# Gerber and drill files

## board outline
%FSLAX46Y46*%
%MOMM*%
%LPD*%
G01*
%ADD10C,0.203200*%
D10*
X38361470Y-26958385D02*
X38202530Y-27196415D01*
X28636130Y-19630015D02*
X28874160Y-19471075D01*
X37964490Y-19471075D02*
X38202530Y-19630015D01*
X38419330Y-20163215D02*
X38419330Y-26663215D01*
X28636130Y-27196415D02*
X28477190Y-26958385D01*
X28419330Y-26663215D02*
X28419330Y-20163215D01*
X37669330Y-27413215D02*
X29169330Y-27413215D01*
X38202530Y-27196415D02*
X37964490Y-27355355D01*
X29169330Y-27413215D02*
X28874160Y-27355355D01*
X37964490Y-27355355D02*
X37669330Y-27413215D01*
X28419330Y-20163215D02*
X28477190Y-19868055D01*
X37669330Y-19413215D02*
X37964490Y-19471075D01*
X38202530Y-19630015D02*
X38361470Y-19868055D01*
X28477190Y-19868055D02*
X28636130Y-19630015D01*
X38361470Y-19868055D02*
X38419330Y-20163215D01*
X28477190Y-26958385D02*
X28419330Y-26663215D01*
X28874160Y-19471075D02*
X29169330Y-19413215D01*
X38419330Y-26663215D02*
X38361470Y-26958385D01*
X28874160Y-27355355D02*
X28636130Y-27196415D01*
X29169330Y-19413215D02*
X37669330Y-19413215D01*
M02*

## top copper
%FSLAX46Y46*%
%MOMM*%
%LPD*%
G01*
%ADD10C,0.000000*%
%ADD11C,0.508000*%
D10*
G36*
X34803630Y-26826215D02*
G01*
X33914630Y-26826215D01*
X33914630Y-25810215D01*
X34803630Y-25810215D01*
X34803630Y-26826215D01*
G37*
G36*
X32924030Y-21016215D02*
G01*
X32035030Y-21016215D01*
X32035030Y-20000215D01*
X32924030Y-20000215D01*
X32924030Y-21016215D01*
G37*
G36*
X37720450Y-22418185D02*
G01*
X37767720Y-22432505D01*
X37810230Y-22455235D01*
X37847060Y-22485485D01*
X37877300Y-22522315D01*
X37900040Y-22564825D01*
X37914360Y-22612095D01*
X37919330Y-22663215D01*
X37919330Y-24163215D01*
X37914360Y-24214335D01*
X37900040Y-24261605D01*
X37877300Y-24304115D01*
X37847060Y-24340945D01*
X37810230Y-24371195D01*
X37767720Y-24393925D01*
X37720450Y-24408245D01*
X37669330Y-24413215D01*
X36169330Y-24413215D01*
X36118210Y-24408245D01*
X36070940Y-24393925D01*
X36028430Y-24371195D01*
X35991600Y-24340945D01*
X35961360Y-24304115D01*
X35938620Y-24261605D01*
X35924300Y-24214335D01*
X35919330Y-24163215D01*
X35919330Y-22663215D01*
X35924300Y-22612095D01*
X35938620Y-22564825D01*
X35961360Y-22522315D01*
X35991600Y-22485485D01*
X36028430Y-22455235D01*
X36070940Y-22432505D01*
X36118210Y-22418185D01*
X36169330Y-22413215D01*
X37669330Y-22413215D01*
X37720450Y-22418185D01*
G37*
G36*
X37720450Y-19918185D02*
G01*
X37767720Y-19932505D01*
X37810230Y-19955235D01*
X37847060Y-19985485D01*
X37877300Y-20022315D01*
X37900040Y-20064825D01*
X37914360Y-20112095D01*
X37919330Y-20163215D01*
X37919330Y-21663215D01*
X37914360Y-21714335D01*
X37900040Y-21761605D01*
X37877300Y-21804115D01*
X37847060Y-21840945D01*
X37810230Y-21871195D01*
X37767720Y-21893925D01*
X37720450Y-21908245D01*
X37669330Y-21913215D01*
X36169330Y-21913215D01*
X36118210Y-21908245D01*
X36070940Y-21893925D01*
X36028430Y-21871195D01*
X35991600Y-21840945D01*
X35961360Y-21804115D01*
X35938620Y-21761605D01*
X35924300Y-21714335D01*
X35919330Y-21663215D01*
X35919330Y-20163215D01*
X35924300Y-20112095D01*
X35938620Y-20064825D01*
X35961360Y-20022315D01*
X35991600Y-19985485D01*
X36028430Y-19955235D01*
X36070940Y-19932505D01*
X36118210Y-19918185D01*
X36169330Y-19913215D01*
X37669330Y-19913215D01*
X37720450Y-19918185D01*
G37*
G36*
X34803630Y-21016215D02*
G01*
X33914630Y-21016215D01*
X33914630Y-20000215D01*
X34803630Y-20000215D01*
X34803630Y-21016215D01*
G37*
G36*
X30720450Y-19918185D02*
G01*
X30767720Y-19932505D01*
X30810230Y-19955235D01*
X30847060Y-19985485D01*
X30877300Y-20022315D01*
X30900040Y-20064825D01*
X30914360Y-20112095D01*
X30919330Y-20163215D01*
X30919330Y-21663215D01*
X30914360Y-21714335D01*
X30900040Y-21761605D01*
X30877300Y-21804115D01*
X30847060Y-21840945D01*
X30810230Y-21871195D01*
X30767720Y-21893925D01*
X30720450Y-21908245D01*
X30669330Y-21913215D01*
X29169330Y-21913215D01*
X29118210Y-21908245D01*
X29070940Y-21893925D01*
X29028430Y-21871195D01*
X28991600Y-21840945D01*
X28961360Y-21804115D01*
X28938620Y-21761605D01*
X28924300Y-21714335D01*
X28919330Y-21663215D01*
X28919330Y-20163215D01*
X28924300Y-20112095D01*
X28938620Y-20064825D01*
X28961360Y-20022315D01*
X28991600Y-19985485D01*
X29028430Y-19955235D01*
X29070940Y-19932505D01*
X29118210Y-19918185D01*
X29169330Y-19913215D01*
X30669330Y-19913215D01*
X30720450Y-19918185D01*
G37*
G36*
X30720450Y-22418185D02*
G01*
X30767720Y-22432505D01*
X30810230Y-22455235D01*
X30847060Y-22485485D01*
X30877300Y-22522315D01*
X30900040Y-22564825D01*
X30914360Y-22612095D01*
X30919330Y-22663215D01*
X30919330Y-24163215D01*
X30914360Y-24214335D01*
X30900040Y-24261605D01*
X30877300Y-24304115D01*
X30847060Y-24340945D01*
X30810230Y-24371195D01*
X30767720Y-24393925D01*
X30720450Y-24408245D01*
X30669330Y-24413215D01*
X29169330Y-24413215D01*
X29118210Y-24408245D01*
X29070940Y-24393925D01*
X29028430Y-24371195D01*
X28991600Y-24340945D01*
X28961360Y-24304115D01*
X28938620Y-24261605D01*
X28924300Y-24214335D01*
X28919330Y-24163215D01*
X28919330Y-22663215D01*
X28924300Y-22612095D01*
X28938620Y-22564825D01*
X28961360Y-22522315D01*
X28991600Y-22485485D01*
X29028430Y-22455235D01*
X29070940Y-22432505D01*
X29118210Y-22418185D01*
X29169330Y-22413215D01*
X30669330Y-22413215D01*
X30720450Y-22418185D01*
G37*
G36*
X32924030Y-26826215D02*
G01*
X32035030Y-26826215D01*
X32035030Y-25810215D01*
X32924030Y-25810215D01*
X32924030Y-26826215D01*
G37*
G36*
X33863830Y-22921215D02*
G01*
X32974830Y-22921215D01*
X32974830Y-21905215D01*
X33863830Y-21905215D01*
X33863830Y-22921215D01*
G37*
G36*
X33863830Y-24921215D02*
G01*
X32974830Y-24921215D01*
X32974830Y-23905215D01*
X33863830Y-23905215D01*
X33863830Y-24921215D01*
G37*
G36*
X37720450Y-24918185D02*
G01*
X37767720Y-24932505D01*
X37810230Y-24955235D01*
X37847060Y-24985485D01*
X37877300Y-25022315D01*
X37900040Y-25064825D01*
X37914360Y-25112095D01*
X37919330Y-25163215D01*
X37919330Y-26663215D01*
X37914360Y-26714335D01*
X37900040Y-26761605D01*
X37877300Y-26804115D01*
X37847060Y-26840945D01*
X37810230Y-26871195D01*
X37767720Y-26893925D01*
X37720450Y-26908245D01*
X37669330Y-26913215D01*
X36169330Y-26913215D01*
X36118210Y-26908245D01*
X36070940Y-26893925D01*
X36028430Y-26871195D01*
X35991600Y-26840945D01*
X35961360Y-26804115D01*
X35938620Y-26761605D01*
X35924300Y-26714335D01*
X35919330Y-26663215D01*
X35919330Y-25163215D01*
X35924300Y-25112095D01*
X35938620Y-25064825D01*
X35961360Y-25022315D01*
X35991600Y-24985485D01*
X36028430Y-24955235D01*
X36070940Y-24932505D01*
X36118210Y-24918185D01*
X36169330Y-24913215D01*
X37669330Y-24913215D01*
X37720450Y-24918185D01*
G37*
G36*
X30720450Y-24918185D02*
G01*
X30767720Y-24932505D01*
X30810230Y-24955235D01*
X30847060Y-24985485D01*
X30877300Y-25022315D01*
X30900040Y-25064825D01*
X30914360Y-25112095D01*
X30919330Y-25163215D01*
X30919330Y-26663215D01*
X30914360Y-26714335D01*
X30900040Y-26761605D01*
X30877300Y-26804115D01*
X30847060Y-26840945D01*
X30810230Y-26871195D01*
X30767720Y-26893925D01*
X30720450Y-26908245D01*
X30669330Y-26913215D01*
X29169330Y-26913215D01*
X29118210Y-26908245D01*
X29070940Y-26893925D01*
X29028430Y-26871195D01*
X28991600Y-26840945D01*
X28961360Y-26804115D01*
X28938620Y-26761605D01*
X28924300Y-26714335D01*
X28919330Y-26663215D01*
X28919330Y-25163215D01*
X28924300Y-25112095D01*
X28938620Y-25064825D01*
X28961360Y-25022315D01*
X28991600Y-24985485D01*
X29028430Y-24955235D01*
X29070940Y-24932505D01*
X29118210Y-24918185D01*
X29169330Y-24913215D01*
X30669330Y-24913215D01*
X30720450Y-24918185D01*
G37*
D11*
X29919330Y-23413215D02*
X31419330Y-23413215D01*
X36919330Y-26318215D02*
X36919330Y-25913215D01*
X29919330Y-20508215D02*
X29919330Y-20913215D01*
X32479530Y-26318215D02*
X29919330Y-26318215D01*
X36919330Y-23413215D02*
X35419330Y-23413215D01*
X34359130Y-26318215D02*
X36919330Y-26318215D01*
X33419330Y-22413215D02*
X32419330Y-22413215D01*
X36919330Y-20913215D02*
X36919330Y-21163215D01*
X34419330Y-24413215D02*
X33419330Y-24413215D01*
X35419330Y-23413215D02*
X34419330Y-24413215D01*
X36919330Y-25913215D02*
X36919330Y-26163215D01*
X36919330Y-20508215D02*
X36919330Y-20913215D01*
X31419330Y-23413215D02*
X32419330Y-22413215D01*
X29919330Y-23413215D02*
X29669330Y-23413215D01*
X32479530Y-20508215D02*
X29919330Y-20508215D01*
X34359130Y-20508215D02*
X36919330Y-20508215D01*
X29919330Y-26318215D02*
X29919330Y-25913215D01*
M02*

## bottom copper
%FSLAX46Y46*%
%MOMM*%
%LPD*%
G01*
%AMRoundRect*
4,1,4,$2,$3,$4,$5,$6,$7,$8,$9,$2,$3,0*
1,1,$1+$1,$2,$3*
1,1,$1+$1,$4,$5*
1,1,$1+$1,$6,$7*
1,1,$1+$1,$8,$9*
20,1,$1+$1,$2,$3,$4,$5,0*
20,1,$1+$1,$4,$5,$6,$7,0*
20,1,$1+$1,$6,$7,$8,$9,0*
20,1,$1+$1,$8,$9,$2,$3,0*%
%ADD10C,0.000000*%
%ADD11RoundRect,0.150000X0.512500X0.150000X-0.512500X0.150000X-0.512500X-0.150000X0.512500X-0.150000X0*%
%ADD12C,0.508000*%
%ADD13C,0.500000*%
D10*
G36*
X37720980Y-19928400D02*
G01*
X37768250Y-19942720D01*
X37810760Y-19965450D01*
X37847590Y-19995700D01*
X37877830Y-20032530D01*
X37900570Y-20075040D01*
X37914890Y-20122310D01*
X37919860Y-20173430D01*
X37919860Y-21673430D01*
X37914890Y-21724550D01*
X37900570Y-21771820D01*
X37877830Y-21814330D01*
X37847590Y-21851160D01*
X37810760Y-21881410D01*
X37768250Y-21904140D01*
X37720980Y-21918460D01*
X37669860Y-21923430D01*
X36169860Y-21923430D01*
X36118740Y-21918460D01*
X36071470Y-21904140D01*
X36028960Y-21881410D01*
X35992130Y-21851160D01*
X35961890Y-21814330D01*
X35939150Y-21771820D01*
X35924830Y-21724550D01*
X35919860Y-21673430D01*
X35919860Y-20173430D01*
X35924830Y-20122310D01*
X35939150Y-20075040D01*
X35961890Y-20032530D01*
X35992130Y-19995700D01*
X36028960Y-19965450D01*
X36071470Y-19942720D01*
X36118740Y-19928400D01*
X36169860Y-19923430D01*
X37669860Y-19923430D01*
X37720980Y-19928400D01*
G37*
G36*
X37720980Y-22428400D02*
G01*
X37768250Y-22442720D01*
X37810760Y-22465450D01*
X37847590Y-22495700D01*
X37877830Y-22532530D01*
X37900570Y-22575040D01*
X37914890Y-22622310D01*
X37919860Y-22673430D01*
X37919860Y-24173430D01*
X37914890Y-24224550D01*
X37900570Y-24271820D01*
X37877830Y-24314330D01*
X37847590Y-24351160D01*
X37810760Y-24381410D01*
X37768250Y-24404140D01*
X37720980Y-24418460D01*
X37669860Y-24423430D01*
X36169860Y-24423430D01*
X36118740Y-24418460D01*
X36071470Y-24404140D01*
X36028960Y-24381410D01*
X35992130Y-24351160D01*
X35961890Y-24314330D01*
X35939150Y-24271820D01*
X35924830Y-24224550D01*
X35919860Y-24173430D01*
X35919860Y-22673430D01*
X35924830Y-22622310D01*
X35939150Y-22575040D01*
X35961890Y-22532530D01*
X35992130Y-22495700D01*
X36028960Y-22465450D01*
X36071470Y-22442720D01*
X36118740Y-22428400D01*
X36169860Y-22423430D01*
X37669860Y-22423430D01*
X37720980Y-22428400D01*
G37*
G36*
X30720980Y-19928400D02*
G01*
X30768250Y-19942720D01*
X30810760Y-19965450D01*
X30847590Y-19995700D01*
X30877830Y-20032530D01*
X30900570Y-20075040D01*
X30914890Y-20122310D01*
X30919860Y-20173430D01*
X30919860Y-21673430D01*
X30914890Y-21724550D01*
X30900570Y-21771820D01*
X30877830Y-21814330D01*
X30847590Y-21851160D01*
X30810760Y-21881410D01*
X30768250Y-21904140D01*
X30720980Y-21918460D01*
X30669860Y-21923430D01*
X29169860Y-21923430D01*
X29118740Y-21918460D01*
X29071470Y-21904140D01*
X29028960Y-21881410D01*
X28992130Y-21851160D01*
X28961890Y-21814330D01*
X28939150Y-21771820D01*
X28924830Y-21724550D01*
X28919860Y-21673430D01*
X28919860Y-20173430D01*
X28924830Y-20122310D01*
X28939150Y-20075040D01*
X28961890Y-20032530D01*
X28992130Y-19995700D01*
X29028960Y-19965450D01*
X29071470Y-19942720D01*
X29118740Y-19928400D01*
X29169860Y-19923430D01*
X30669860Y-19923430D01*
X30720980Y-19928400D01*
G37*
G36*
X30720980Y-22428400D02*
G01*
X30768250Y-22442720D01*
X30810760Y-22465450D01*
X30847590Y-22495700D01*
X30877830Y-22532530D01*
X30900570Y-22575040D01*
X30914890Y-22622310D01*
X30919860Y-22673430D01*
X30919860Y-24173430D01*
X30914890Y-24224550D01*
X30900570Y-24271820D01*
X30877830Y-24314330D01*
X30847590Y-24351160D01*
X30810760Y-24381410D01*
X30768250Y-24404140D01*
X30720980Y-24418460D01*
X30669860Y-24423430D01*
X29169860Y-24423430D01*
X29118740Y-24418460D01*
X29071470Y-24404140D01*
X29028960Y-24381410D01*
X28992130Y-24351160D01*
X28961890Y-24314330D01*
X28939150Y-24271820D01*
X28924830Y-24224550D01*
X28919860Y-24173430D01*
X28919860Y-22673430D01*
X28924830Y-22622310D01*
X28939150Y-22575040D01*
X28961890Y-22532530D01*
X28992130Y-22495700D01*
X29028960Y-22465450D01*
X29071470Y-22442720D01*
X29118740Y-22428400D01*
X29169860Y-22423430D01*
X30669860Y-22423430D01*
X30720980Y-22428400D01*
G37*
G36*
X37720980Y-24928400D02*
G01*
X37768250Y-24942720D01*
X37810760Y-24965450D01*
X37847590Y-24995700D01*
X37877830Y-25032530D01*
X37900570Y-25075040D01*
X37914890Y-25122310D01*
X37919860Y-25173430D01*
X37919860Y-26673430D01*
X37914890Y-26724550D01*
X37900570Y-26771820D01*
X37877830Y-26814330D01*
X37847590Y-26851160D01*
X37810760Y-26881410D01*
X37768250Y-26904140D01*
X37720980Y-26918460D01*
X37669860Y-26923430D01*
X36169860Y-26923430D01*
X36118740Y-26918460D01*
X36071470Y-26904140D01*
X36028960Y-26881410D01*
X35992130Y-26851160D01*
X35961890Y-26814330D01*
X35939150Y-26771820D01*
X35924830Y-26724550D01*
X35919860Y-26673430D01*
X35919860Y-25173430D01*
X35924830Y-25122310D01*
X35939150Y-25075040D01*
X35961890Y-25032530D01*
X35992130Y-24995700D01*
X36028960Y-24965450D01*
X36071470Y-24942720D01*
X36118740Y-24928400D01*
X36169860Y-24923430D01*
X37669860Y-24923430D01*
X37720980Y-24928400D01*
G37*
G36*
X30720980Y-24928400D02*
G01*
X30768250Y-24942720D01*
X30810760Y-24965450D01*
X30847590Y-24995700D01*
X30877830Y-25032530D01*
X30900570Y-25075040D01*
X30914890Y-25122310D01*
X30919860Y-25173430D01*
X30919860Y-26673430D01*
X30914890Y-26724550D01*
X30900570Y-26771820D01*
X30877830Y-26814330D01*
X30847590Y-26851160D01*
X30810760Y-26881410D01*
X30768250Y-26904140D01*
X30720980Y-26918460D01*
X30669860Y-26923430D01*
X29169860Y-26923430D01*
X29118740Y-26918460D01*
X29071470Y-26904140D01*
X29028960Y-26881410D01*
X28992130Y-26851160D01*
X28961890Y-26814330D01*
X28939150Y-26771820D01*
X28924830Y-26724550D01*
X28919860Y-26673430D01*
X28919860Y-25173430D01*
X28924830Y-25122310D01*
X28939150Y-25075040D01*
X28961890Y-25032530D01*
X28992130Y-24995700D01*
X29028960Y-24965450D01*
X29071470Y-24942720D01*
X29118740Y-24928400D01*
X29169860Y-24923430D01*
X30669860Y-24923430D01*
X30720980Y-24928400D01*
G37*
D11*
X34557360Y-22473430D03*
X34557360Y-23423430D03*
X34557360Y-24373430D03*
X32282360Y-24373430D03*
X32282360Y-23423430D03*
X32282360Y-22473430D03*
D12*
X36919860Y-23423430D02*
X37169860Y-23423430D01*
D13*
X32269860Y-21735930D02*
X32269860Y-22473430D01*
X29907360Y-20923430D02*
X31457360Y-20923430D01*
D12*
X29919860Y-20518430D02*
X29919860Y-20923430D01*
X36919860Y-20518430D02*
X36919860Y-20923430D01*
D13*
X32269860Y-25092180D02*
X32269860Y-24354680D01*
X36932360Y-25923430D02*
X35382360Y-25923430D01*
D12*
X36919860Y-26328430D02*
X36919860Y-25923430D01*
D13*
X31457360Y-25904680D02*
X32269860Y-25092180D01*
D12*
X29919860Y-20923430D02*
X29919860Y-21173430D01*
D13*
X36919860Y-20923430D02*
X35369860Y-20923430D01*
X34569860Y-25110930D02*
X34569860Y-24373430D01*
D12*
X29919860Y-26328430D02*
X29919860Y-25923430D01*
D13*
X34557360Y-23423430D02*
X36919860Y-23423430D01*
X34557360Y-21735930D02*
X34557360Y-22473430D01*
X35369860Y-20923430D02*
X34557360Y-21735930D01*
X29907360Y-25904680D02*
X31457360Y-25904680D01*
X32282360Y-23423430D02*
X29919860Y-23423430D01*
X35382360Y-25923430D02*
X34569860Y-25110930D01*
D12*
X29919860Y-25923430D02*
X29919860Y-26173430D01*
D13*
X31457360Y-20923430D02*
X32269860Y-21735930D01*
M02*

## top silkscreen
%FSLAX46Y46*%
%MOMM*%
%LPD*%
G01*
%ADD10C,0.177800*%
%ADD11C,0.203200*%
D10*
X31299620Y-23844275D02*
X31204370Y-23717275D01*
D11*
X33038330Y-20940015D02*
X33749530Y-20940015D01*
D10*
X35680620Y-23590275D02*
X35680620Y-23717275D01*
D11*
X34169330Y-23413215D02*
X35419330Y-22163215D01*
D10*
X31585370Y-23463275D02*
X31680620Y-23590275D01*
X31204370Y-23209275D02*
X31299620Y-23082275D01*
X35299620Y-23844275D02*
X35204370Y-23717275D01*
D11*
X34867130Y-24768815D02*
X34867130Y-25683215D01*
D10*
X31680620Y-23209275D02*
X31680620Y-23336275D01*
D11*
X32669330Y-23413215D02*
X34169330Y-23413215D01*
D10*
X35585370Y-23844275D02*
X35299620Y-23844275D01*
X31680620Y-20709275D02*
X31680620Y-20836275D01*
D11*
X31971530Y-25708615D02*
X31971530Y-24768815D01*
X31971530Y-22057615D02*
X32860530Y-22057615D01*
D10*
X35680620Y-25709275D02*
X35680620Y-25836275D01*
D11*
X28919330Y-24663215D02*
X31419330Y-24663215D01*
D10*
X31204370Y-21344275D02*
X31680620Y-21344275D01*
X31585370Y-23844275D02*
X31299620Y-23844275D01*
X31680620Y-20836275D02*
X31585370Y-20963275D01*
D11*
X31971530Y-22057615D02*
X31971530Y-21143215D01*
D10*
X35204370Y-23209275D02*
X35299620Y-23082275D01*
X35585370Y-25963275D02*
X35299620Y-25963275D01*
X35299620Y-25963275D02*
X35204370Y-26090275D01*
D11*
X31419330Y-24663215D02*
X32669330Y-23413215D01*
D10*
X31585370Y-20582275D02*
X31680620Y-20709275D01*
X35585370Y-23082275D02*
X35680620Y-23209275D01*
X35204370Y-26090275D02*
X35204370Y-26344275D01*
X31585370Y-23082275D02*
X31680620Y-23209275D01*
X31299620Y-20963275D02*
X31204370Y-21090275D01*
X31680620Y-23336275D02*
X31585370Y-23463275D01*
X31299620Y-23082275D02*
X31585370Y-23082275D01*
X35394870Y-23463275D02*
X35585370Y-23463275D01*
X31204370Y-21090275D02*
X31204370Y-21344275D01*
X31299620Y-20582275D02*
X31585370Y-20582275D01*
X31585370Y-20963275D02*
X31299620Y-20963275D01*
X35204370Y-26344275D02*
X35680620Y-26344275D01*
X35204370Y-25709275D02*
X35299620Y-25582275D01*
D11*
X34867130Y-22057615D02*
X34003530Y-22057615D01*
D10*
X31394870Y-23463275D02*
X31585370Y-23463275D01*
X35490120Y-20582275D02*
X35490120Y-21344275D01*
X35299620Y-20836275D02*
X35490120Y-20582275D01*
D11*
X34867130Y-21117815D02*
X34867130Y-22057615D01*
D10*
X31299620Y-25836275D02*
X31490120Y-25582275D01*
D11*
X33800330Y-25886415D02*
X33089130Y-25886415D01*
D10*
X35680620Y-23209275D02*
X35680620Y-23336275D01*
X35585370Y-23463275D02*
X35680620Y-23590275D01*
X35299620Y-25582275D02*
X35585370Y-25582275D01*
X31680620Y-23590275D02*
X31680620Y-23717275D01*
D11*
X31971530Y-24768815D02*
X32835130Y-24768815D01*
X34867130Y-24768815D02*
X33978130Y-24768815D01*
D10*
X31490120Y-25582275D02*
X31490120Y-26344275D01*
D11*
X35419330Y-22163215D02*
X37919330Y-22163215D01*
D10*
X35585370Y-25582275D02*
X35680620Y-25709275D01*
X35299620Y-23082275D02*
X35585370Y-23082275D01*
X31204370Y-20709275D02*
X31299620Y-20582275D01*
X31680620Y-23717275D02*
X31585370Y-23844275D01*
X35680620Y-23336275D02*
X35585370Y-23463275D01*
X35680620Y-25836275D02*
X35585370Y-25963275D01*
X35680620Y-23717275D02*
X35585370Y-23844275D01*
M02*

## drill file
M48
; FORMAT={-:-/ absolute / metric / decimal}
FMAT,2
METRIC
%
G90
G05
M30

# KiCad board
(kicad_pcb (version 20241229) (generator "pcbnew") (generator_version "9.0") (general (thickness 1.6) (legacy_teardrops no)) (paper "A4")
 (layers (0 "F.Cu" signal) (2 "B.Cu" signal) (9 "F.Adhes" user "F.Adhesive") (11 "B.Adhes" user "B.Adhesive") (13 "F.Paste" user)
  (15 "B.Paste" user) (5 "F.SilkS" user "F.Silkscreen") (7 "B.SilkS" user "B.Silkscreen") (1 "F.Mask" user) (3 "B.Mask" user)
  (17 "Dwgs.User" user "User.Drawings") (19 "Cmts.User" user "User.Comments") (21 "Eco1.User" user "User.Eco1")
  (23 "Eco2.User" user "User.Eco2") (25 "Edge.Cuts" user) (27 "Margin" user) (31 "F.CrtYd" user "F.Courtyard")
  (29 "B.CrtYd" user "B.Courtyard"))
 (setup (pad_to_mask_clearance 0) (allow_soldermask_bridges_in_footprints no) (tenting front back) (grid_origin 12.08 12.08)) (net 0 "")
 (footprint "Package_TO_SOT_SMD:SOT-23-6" (layer "B.Cu") (at 33.41986 23.42343 180)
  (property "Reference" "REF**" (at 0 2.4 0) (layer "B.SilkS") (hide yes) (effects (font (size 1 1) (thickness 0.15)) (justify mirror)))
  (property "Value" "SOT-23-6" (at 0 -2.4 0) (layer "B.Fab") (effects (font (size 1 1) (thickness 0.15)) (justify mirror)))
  (pad "1" smd roundrect (at -1.1375 0.95 180) (size 1.325 0.6) (layers "B.Cu" "B.Mask" "B.Paste") (roundrect_rratio 0.25))
  (pad "2" smd roundrect (at -1.1375 0 180) (size 1.325 0.6) (layers "B.Cu" "B.Mask" "B.Paste") (roundrect_rratio 0.25))
  (pad "3" smd roundrect (at -1.1375 -0.95 180) (size 1.325 0.6) (layers "B.Cu" "B.Mask" "B.Paste") (roundrect_rratio 0.25))
  (pad "4" smd roundrect (at 1.1375 -0.95 180) (size 1.325 0.6) (layers "B.Cu" "B.Mask" "B.Paste") (roundrect_rratio 0.25))
  (pad "5" smd roundrect (at 1.1375 0 180) (size 1.325 0.6) (layers "B.Cu" "B.Mask" "B.Paste") (roundrect_rratio 0.25))
  (pad "6" smd roundrect (at 1.1375 0.95 180) (size 1.325 0.6) (layers "B.Cu" "B.Mask" "B.Paste") (roundrect_rratio 0.25)))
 (gr_poly
  (pts (xy 34.80363 25.810215) (xy 33.91463 25.810215) (xy 33.91463 26.826215) (xy 34.80363 26.826215)) (stroke (width 0) (type solid))
  (fill yes) (layer "F.Cu"))
 (gr_poly
  (pts (xy 32.92403 20.000215) (xy 32.03503 20.000215) (xy 32.03503 21.016215) (xy 32.92403 21.016215)) (stroke (width 0) (type solid))
  (fill yes) (layer "F.Cu"))
 (gr_poly
  (pts (xy 37.72045 24.408245) (xy 37.76772 24.393925) (xy 37.81023 24.371195) (xy 37.84706 24.340945) (xy 37.8773 24.304115)
   (xy 37.90004 24.261605) (xy 37.91436 24.214335) (xy 37.91933 24.163215) (xy 37.91933 22.663215) (xy 37.91436 22.612095)
   (xy 37.90004 22.564825) (xy 37.8773 22.522315) (xy 37.84706 22.485485) (xy 37.81023 22.455235) (xy 37.76772 22.432505)
   (xy 37.72045 22.418185) (xy 37.66933 22.413215) (xy 36.16933 22.413215) (xy 36.11821 22.418185) (xy 36.07094 22.432505)
   (xy 36.02843 22.455235) (xy 35.9916 22.485485) (xy 35.96136 22.522315) (xy 35.93862 22.564825) (xy 35.9243 22.612095)
   (xy 35.91933 22.663215) (xy 35.91933 24.163215) (xy 35.9243 24.214335) (xy 35.93862 24.261605) (xy 35.96136 24.304115)
   (xy 35.9916 24.340945) (xy 36.02843 24.371195) (xy 36.07094 24.393925) (xy 36.11821 24.408245) (xy 36.16933 24.413215)
   (xy 37.66933 24.413215))
  (stroke (width 0) (type solid)) (fill yes) (layer "F.Cu"))
 (gr_poly
  (pts (xy 37.72045 21.908245) (xy 37.76772 21.893925) (xy 37.81023 21.871195) (xy 37.84706 21.840945) (xy 37.8773 21.804115)
   (xy 37.90004 21.761605) (xy 37.91436 21.714335) (xy 37.91933 21.663215) (xy 37.91933 20.163215) (xy 37.91436 20.112095)
   (xy 37.90004 20.064825) (xy 37.8773 20.022315) (xy 37.84706 19.985485) (xy 37.81023 19.955235) (xy 37.76772 19.932505)
   (xy 37.72045 19.918185) (xy 37.66933 19.913215) (xy 36.16933 19.913215) (xy 36.11821 19.918185) (xy 36.07094 19.932505)
   (xy 36.02843 19.955235) (xy 35.9916 19.985485) (xy 35.96136 20.022315) (xy 35.93862 20.064825) (xy 35.9243 20.112095)
   (xy 35.91933 20.163215) (xy 35.91933 21.663215) (xy 35.9243 21.714335) (xy 35.93862 21.761605) (xy 35.96136 21.804115)
   (xy 35.9916 21.840945) (xy 36.02843 21.871195) (xy 36.07094 21.893925) (xy 36.11821 21.908245) (xy 36.16933 21.913215)
   (xy 37.66933 21.913215))
  (stroke (width 0) (type solid)) (fill yes) (layer "F.Cu"))
 (gr_poly
  (pts (xy 34.80363 20.000215) (xy 33.91463 20.000215) (xy 33.91463 21.016215) (xy 34.80363 21.016215)) (stroke (width 0) (type solid))
  (fill yes) (layer "F.Cu"))
 (gr_poly
  (pts (xy 30.72045 21.908245) (xy 30.76772 21.893925) (xy 30.81023 21.871195) (xy 30.84706 21.840945) (xy 30.8773 21.804115)
   (xy 30.90004 21.761605) (xy 30.91436 21.714335) (xy 30.91933 21.663215) (xy 30.91933 20.163215) (xy 30.91436 20.112095)
   (xy 30.90004 20.064825) (xy 30.8773 20.022315) (xy 30.84706 19.985485) (xy 30.81023 19.955235) (xy 30.76772 19.932505)
   (xy 30.72045 19.918185) (xy 30.66933 19.913215) (xy 29.16933 19.913215) (xy 29.11821 19.918185) (xy 29.07094 19.932505)
   (xy 29.02843 19.955235) (xy 28.9916 19.985485) (xy 28.96136 20.022315) (xy 28.93862 20.064825) (xy 28.9243 20.112095)
   (xy 28.91933 20.163215) (xy 28.91933 21.663215) (xy 28.9243 21.714335) (xy 28.93862 21.761605) (xy 28.96136 21.804115)
   (xy 28.9916 21.840945) (xy 29.02843 21.871195) (xy 29.07094 21.893925) (xy 29.11821 21.908245) (xy 29.16933 21.913215)
   (xy 30.66933 21.913215))
  (stroke (width 0) (type solid)) (fill yes) (layer "F.Cu"))
 (gr_poly
  (pts (xy 30.72045 24.408245) (xy 30.76772 24.393925) (xy 30.81023 24.371195) (xy 30.84706 24.340945) (xy 30.8773 24.304115)
   (xy 30.90004 24.261605) (xy 30.91436 24.214335) (xy 30.91933 24.163215) (xy 30.91933 22.663215) (xy 30.91436 22.612095)
   (xy 30.90004 22.564825) (xy 30.8773 22.522315) (xy 30.84706 22.485485) (xy 30.81023 22.455235) (xy 30.76772 22.432505)
   (xy 30.72045 22.418185) (xy 30.66933 22.413215) (xy 29.16933 22.413215) (xy 29.11821 22.418185) (xy 29.07094 22.432505)
   (xy 29.02843 22.455235) (xy 28.9916 22.485485) (xy 28.96136 22.522315) (xy 28.93862 22.564825) (xy 28.9243 22.612095)
   (xy 28.91933 22.663215) (xy 28.91933 24.163215) (xy 28.9243 24.214335) (xy 28.93862 24.261605) (xy 28.96136 24.304115)
   (xy 28.9916 24.340945) (xy 29.02843 24.371195) (xy 29.07094 24.393925) (xy 29.11821 24.408245) (xy 29.16933 24.413215)
   (xy 30.66933 24.413215))
  (stroke (width 0) (type solid)) (fill yes) (layer "F.Cu"))
 (gr_poly
  (pts (xy 32.92403 25.810215) (xy 32.03503 25.810215) (xy 32.03503 26.826215) (xy 32.92403 26.826215)) (stroke (width 0) (type solid))
  (fill yes) (layer "F.Cu"))
 (gr_poly
  (pts (xy 33.86383 21.905215) (xy 32.97483 21.905215) (xy 32.97483 22.921215) (xy 33.86383 22.921215)) (stroke (width 0) (type solid))
  (fill yes) (layer "F.Cu"))
 (gr_poly
  (pts (xy 33.86383 23.905215) (xy 32.97483 23.905215) (xy 32.97483 24.921215) (xy 33.86383 24.921215)) (stroke (width 0) (type solid))
  (fill yes) (layer "F.Cu"))
 (gr_poly
  (pts (xy 37.72045 26.908245) (xy 37.76772 26.893925) (xy 37.81023 26.871195) (xy 37.84706 26.840945) (xy 37.8773 26.804115)
   (xy 37.90004 26.761605) (xy 37.91436 26.714335) (xy 37.91933 26.663215) (xy 37.91933 25.163215) (xy 37.91436 25.112095)
   (xy 37.90004 25.064825) (xy 37.8773 25.022315) (xy 37.84706 24.985485) (xy 37.81023 24.955235) (xy 37.76772 24.932505)
   (xy 37.72045 24.918185) (xy 37.66933 24.913215) (xy 36.16933 24.913215) (xy 36.11821 24.918185) (xy 36.07094 24.932505)
   (xy 36.02843 24.955235) (xy 35.9916 24.985485) (xy 35.96136 25.022315) (xy 35.93862 25.064825) (xy 35.9243 25.112095)
   (xy 35.91933 25.163215) (xy 35.91933 26.663215) (xy 35.9243 26.714335) (xy 35.93862 26.761605) (xy 35.96136 26.804115)
   (xy 35.9916 26.840945) (xy 36.02843 26.871195) (xy 36.07094 26.893925) (xy 36.11821 26.908245) (xy 36.16933 26.913215)
   (xy 37.66933 26.913215))
  (stroke (width 0) (type solid)) (fill yes) (layer "F.Cu"))
 (gr_poly
  (pts (xy 30.72045 26.908245) (xy 30.76772 26.893925) (xy 30.81023 26.871195) (xy 30.84706 26.840945) (xy 30.8773 26.804115)
   (xy 30.90004 26.761605) (xy 30.91436 26.714335) (xy 30.91933 26.663215) (xy 30.91933 25.163215) (xy 30.91436 25.112095)
   (xy 30.90004 25.064825) (xy 30.8773 25.022315) (xy 30.84706 24.985485) (xy 30.81023 24.955235) (xy 30.76772 24.932505)
   (xy 30.72045 24.918185) (xy 30.66933 24.913215) (xy 29.16933 24.913215) (xy 29.11821 24.918185) (xy 29.07094 24.932505)
   (xy 29.02843 24.955235) (xy 28.9916 24.985485) (xy 28.96136 25.022315) (xy 28.93862 25.064825) (xy 28.9243 25.112095)
   (xy 28.91933 25.163215) (xy 28.91933 26.663215) (xy 28.9243 26.714335) (xy 28.93862 26.761605) (xy 28.96136 26.804115)
   (xy 28.9916 26.840945) (xy 29.02843 26.871195) (xy 29.07094 26.893925) (xy 29.11821 26.908245) (xy 29.16933 26.913215)
   (xy 30.66933 26.913215))
  (stroke (width 0) (type solid)) (fill yes) (layer "F.Cu"))
 (gr_poly
  (pts (xy 36.11874 21.91846) (xy 36.07147 21.90414) (xy 36.02896 21.88141) (xy 35.99213 21.85116) (xy 35.96189 21.81433)
   (xy 35.93915 21.77182) (xy 35.92483 21.72455) (xy 35.91986 21.67343) (xy 35.91986 20.17343) (xy 35.92483 20.12231) (xy 35.93915 20.07504)
   (xy 35.96189 20.03253) (xy 35.99213 19.9957) (xy 36.02896 19.96545) (xy 36.07147 19.94272) (xy 36.11874 19.9284) (xy 36.16986 19.92343)
   (xy 37.66986 19.92343) (xy 37.72098 19.9284) (xy 37.76825 19.94272) (xy 37.81076 19.96545) (xy 37.84759 19.9957) (xy 37.87783 20.03253)
   (xy 37.90057 20.07504) (xy 37.91489 20.12231) (xy 37.91986 20.17343) (xy 37.91986 21.67343) (xy 37.91489 21.72455) (xy 37.90057 21.77182)
   (xy 37.87783 21.81433) (xy 37.84759 21.85116) (xy 37.81076 21.88141) (xy 37.76825 21.90414) (xy 37.72098 21.91846) (xy 37.66986 21.92343)
   (xy 36.16986 21.92343))
  (stroke (width 0) (type solid)) (fill yes) (layer "B.Cu"))
 (gr_poly
  (pts (xy 36.11874 24.41846) (xy 36.07147 24.40414) (xy 36.02896 24.38141) (xy 35.99213 24.35116) (xy 35.96189 24.31433)
   (xy 35.93915 24.27182) (xy 35.92483 24.22455) (xy 35.91986 24.17343) (xy 35.91986 22.67343) (xy 35.92483 22.62231) (xy 35.93915 22.57504)
   (xy 35.96189 22.53253) (xy 35.99213 22.4957) (xy 36.02896 22.46545) (xy 36.07147 22.44272) (xy 36.11874 22.4284) (xy 36.16986 22.42343)
   (xy 37.66986 22.42343) (xy 37.72098 22.4284) (xy 37.76825 22.44272) (xy 37.81076 22.46545) (xy 37.84759 22.4957) (xy 37.87783 22.53253)
   (xy 37.90057 22.57504) (xy 37.91489 22.62231) (xy 37.91986 22.67343) (xy 37.91986 24.17343) (xy 37.91489 24.22455) (xy 37.90057 24.27182)
   (xy 37.87783 24.31433) (xy 37.84759 24.35116) (xy 37.81076 24.38141) (xy 37.76825 24.40414) (xy 37.72098 24.41846) (xy 37.66986 24.42343)
   (xy 36.16986 24.42343))
  (stroke (width 0) (type solid)) (fill yes) (layer "B.Cu"))
 (gr_poly
  (pts (xy 29.11874 21.91846) (xy 29.07147 21.90414) (xy 29.02896 21.88141) (xy 28.99213 21.85116) (xy 28.96189 21.81433)
   (xy 28.93915 21.77182) (xy 28.92483 21.72455) (xy 28.91986 21.67343) (xy 28.91986 20.17343) (xy 28.92483 20.12231) (xy 28.93915 20.07504)
   (xy 28.96189 20.03253) (xy 28.99213 19.9957) (xy 29.02896 19.96545) (xy 29.07147 19.94272) (xy 29.11874 19.9284) (xy 29.16986 19.92343)
   (xy 30.66986 19.92343) (xy 30.72098 19.9284) (xy 30.76825 19.94272) (xy 30.81076 19.96545) (xy 30.84759 19.9957) (xy 30.87783 20.03253)
   (xy 30.90057 20.07504) (xy 30.91489 20.12231) (xy 30.91986 20.17343) (xy 30.91986 21.67343) (xy 30.91489 21.72455) (xy 30.90057 21.77182)
   (xy 30.87783 21.81433) (xy 30.84759 21.85116) (xy 30.81076 21.88141) (xy 30.76825 21.90414) (xy 30.72098 21.91846) (xy 30.66986 21.92343)
   (xy 29.16986 21.92343))
  (stroke (width 0) (type solid)) (fill yes) (layer "B.Cu"))
 (gr_poly
  (pts (xy 29.11874 24.41846) (xy 29.07147 24.40414) (xy 29.02896 24.38141) (xy 28.99213 24.35116) (xy 28.96189 24.31433)
   (xy 28.93915 24.27182) (xy 28.92483 24.22455) (xy 28.91986 24.17343) (xy 28.91986 22.67343) (xy 28.92483 22.62231) (xy 28.93915 22.57504)
   (xy 28.96189 22.53253) (xy 28.99213 22.4957) (xy 29.02896 22.46545) (xy 29.07147 22.44272) (xy 29.11874 22.4284) (xy 29.16986 22.42343)
   (xy 30.66986 22.42343) (xy 30.72098 22.4284) (xy 30.76825 22.44272) (xy 30.81076 22.46545) (xy 30.84759 22.4957) (xy 30.87783 22.53253)
   (xy 30.90057 22.57504) (xy 30.91489 22.62231) (xy 30.91986 22.67343) (xy 30.91986 24.17343) (xy 30.91489 24.22455) (xy 30.90057 24.27182)
   (xy 30.87783 24.31433) (xy 30.84759 24.35116) (xy 30.81076 24.38141) (xy 30.76825 24.40414) (xy 30.72098 24.41846) (xy 30.66986 24.42343)
   (xy 29.16986 24.42343))
  (stroke (width 0) (type solid)) (fill yes) (layer "B.Cu"))
 (gr_poly
  (pts (xy 36.11874 26.91846) (xy 36.07147 26.90414) (xy 36.02896 26.88141) (xy 35.99213 26.85116) (xy 35.96189 26.81433)
   (xy 35.93915 26.77182) (xy 35.92483 26.72455) (xy 35.91986 26.67343) (xy 35.91986 25.17343) (xy 35.92483 25.12231) (xy 35.93915 25.07504)
   (xy 35.96189 25.03253) (xy 35.99213 24.9957) (xy 36.02896 24.96545) (xy 36.07147 24.94272) (xy 36.11874 24.9284) (xy 36.16986 24.92343)
   (xy 37.66986 24.92343) (xy 37.72098 24.9284) (xy 37.76825 24.94272) (xy 37.81076 24.96545) (xy 37.84759 24.9957) (xy 37.87783 25.03253)
   (xy 37.90057 25.07504) (xy 37.91489 25.12231) (xy 37.91986 25.17343) (xy 37.91986 26.67343) (xy 37.91489 26.72455) (xy 37.90057 26.77182)
   (xy 37.87783 26.81433) (xy 37.84759 26.85116) (xy 37.81076 26.88141) (xy 37.76825 26.90414) (xy 37.72098 26.91846) (xy 37.66986 26.92343)
   (xy 36.16986 26.92343))
  (stroke (width 0) (type solid)) (fill yes) (layer "B.Cu"))
 (gr_poly
  (pts (xy 29.11874 26.91846) (xy 29.07147 26.90414) (xy 29.02896 26.88141) (xy 28.99213 26.85116) (xy 28.96189 26.81433)
   (xy 28.93915 26.77182) (xy 28.92483 26.72455) (xy 28.91986 26.67343) (xy 28.91986 25.17343) (xy 28.92483 25.12231) (xy 28.93915 25.07504)
   (xy 28.96189 25.03253) (xy 28.99213 24.9957) (xy 29.02896 24.96545) (xy 29.07147 24.94272) (xy 29.11874 24.9284) (xy 29.16986 24.92343)
   (xy 30.66986 24.92343) (xy 30.72098 24.9284) (xy 30.76825 24.94272) (xy 30.81076 24.96545) (xy 30.84759 24.9957) (xy 30.87783 25.03253)
   (xy 30.90057 25.07504) (xy 30.91489 25.12231) (xy 30.91986 25.17343) (xy 30.91986 26.67343) (xy 30.91489 26.72455) (xy 30.90057 26.77182)
   (xy 30.87783 26.81433) (xy 30.84759 26.85116) (xy 30.81076 26.88141) (xy 30.76825 26.90414) (xy 30.72098 26.91846) (xy 30.66986 26.92343)
   (xy 29.16986 26.92343))
  (stroke (width 0) (type solid)) (fill yes) (layer "B.Cu"))
 (gr_line (start 31.29962 23.844275) (end 31.20437 23.717275) (stroke (width 0.1778) (type solid)) (layer "F.SilkS"))
 (gr_line (start 33.03833 20.940015) (end 33.74953 20.940015) (stroke (width 0.2032) (type solid)) (layer "F.SilkS"))
 (gr_line (start 35.68062 23.590275) (end 35.68062 23.717275) (stroke (width 0.1778) (type solid)) (layer "F.SilkS"))
 (gr_line (start 34.16933 23.413215) (end 35.41933 22.163215) (stroke (width 0.2032) (type solid)) (layer "F.SilkS"))
 (gr_line (start 31.58537 23.463275) (end 31.68062 23.590275) (stroke (width 0.1778) (type solid)) (layer "F.SilkS"))
 (gr_line (start 31.20437 23.209275) (end 31.29962 23.082275) (stroke (width 0.1778) (type solid)) (layer "F.SilkS"))
 (gr_line (start 35.29962 23.844275) (end 35.20437 23.717275) (stroke (width 0.1778) (type solid)) (layer "F.SilkS"))
 (gr_line (start 34.86713 24.768815) (end 34.86713 25.683215) (stroke (width 0.2032) (type solid)) (layer "F.SilkS"))
 (gr_line (start 31.68062 23.209275) (end 31.68062 23.336275) (stroke (width 0.1778) (type solid)) (layer "F.SilkS"))
 (gr_line (start 32.66933 23.413215) (end 34.16933 23.413215) (stroke (width 0.2032) (type solid)) (layer "F.SilkS"))
 (gr_line (start 35.58537 23.844275) (end 35.29962 23.844275) (stroke (width 0.1778) (type solid)) (layer "F.SilkS"))
 (gr_line (start 31.68062 20.709275) (end 31.68062 20.836275) (stroke (width 0.1778) (type solid)) (layer "F.SilkS"))
 (gr_line (start 31.97153 25.708615) (end 31.97153 24.768815) (stroke (width 0.2032) (type solid)) (layer "F.SilkS"))
 (gr_line (start 31.97153 22.057615) (end 32.86053 22.057615) (stroke (width 0.2032) (type solid)) (layer "F.SilkS"))
 (gr_line (start 35.68062 25.709275) (end 35.68062 25.836275) (stroke (width 0.1778) (type solid)) (layer "F.SilkS"))
 (gr_line (start 28.91933 24.663215) (end 31.41933 24.663215) (stroke (width 0.2032) (type solid)) (layer "F.SilkS"))
 (gr_line (start 31.20437 21.344275) (end 31.68062 21.344275) (stroke (width 0.1778) (type solid)) (layer "F.SilkS"))
 (gr_line (start 31.58537 23.844275) (end 31.29962 23.844275) (stroke (width 0.1778) (type solid)) (layer "F.SilkS"))
 (gr_line (start 31.68062 20.836275) (end 31.58537 20.963275) (stroke (width 0.1778) (type solid)) (layer "F.SilkS"))
 (gr_line (start 31.97153 22.057615) (end 31.97153 21.143215) (stroke (width 0.2032) (type solid)) (layer "F.SilkS"))
 (gr_line (start 35.20437 23.209275) (end 35.29962 23.082275) (stroke (width 0.1778) (type solid)) (layer "F.SilkS"))
 (gr_line (start 35.58537 25.963275) (end 35.29962 25.963275) (stroke (width 0.1778) (type solid)) (layer "F.SilkS"))
 (gr_line (start 35.29962 25.963275) (end 35.20437 26.090275) (stroke (width 0.1778) (type solid)) (layer "F.SilkS"))
 (gr_line (start 31.41933 24.663215) (end 32.66933 23.413215) (stroke (width 0.2032) (type solid)) (layer "F.SilkS"))
 (gr_line (start 31.58537 20.582275) (end 31.68062 20.709275) (stroke (width 0.1778) (type solid)) (layer "F.SilkS"))
 (gr_line (start 35.58537 23.082275) (end 35.68062 23.209275) (stroke (width 0.1778) (type solid)) (layer "F.SilkS"))
 (gr_line (start 35.20437 26.090275) (end 35.20437 26.344275) (stroke (width 0.1778) (type solid)) (layer "F.SilkS"))
 (gr_line (start 31.58537 23.082275) (end 31.68062 23.209275) (stroke (width 0.1778) (type solid)) (layer "F.SilkS"))
 (gr_line (start 31.29962 20.963275) (end 31.20437 21.090275) (stroke (width 0.1778) (type solid)) (layer "F.SilkS"))
 (gr_line (start 31.68062 23.336275) (end 31.58537 23.463275) (stroke (width 0.1778) (type solid)) (layer "F.SilkS"))
 (gr_line (start 31.29962 23.082275) (end 31.58537 23.082275) (stroke (width 0.1778) (type solid)) (layer "F.SilkS"))
 (gr_line (start 35.39487 23.463275) (end 35.58537 23.463275) (stroke (width 0.1778) (type solid)) (layer "F.SilkS"))
 (gr_line (start 31.20437 21.090275) (end 31.20437 21.344275) (stroke (width 0.1778) (type solid)) (layer "F.SilkS"))
 (gr_line (start 31.29962 20.582275) (end 31.58537 20.582275) (stroke (width 0.1778) (type solid)) (layer "F.SilkS"))
 (gr_line (start 31.58537 20.963275) (end 31.29962 20.963275) (stroke (width 0.1778) (type solid)) (layer "F.SilkS"))
 (gr_line (start 35.20437 26.344275) (end 35.68062 26.344275) (stroke (width 0.1778) (type solid)) (layer "F.SilkS"))
 (gr_line (start 35.20437 25.709275) (end 35.29962 25.582275) (stroke (width 0.1778) (type solid)) (layer "F.SilkS"))
 (gr_line (start 34.86713 22.057615) (end 34.00353 22.057615) (stroke (width 0.2032) (type solid)) (layer "F.SilkS"))
 (gr_line (start 31.39487 23.463275) (end 31.58537 23.463275) (stroke (width 0.1778) (type solid)) (layer "F.SilkS"))
 (gr_line (start 35.49012 20.582275) (end 35.49012 21.344275) (stroke (width 0.1778) (type solid)) (layer "F.SilkS"))
 (gr_line (start 35.29962 20.836275) (end 35.49012 20.582275) (stroke (width 0.1778) (type solid)) (layer "F.SilkS"))
 (gr_line (start 34.86713 21.117815) (end 34.86713 22.057615) (stroke (width 0.2032) (type solid)) (layer "F.SilkS"))
 (gr_line (start 31.29962 25.836275) (end 31.49012 25.582275) (stroke (width 0.1778) (type solid)) (layer "F.SilkS"))
 (gr_line (start 33.80033 25.886415) (end 33.08913 25.886415) (stroke (width 0.2032) (type solid)) (layer "F.SilkS"))
 (gr_line (start 35.68062 23.209275) (end 35.68062 23.336275) (stroke (width 0.1778) (type solid)) (layer "F.SilkS"))
 (gr_line (start 35.58537 23.463275) (end 35.68062 23.590275) (stroke (width 0.1778) (type solid)) (layer "F.SilkS"))
 (gr_line (start 35.29962 25.582275) (end 35.58537 25.582275) (stroke (width 0.1778) (type solid)) (layer "F.SilkS"))
 (gr_line (start 31.68062 23.590275) (end 31.68062 23.717275) (stroke (width 0.1778) (type solid)) (layer "F.SilkS"))
 (gr_line (start 31.97153 24.768815) (end 32.83513 24.768815) (stroke (width 0.2032) (type solid)) (layer "F.SilkS"))
 (gr_line (start 34.86713 24.768815) (end 33.97813 24.768815) (stroke (width 0.2032) (type solid)) (layer "F.SilkS"))
 (gr_line (start 31.49012 25.582275) (end 31.49012 26.344275) (stroke (width 0.1778) (type solid)) (layer "F.SilkS"))
 (gr_line (start 35.41933 22.163215) (end 37.91933 22.163215) (stroke (width 0.2032) (type solid)) (layer "F.SilkS"))
 (gr_line (start 35.58537 25.582275) (end 35.68062 25.709275) (stroke (width 0.1778) (type solid)) (layer "F.SilkS"))
 (gr_line (start 35.29962 23.082275) (end 35.58537 23.082275) (stroke (width 0.1778) (type solid)) (layer "F.SilkS"))
 (gr_line (start 31.20437 20.709275) (end 31.29962 20.582275) (stroke (width 0.1778) (type solid)) (layer "F.SilkS"))
 (gr_line (start 31.68062 23.717275) (end 31.58537 23.844275) (stroke (width 0.1778) (type solid)) (layer "F.SilkS"))
 (gr_line (start 35.68062 23.336275) (end 35.58537 23.463275) (stroke (width 0.1778) (type solid)) (layer "F.SilkS"))
 (gr_line (start 35.68062 25.836275) (end 35.58537 25.963275) (stroke (width 0.1778) (type solid)) (layer "F.SilkS"))
 (gr_line (start 35.68062 23.717275) (end 35.58537 23.844275) (stroke (width 0.1778) (type solid)) (layer "F.SilkS"))
 (gr_line (start 38.36147 26.958385) (end 38.20253 27.196415) (stroke (width 0.2032) (type solid)) (layer "Edge.Cuts"))
 (gr_line (start 28.63613 19.630015) (end 28.87416 19.471075) (stroke (width 0.2032) (type solid)) (layer "Edge.Cuts"))
 (gr_line (start 37.96449 19.471075) (end 38.20253 19.630015) (stroke (width 0.2032) (type solid)) (layer "Edge.Cuts"))
 (gr_line (start 38.41933 20.163215) (end 38.41933 26.663215) (stroke (width 0.2032) (type solid)) (layer "Edge.Cuts"))
 (gr_line (start 28.63613 27.196415) (end 28.47719 26.958385) (stroke (width 0.2032) (type solid)) (layer "Edge.Cuts"))
 (gr_line (start 28.41933 26.663215) (end 28.41933 20.163215) (stroke (width 0.2032) (type solid)) (layer "Edge.Cuts"))
 (gr_line (start 37.66933 27.413215) (end 29.16933 27.413215) (stroke (width 0.2032) (type solid)) (layer "Edge.Cuts"))
 (gr_line (start 38.20253 27.196415) (end 37.96449 27.355355) (stroke (width 0.2032) (type solid)) (layer "Edge.Cuts"))
 (gr_line (start 29.16933 27.413215) (end 28.87416 27.355355) (stroke (width 0.2032) (type solid)) (layer "Edge.Cuts"))
 (gr_line (start 37.96449 27.355355) (end 37.66933 27.413215) (stroke (width 0.2032) (type solid)) (layer "Edge.Cuts"))
 (gr_line (start 28.41933 20.163215) (end 28.47719 19.868055) (stroke (width 0.2032) (type solid)) (layer "Edge.Cuts"))
 (gr_line (start 37.66933 19.413215) (end 37.96449 19.471075) (stroke (width 0.2032) (type solid)) (layer "Edge.Cuts"))
 (gr_line (start 38.20253 19.630015) (end 38.36147 19.868055) (stroke (width 0.2032) (type solid)) (layer "Edge.Cuts"))
 (gr_line (start 28.47719 19.868055) (end 28.63613 19.630015) (stroke (width 0.2032) (type solid)) (layer "Edge.Cuts"))
 (gr_line (start 38.36147 19.868055) (end 38.41933 20.163215) (stroke (width 0.2032) (type solid)) (layer "Edge.Cuts"))
 (gr_line (start 28.47719 26.958385) (end 28.41933 26.663215) (stroke (width 0.2032) (type solid)) (layer "Edge.Cuts"))
 (gr_line (start 28.87416 19.471075) (end 29.16933 19.413215) (stroke (width 0.2032) (type solid)) (layer "Edge.Cuts"))
 (gr_line (start 38.41933 26.663215) (end 38.36147 26.958385) (stroke (width 0.2032) (type solid)) (layer "Edge.Cuts"))
 (gr_line (start 28.87416 27.355355) (end 28.63613 27.196415) (stroke (width 0.2032) (type solid)) (layer "Edge.Cuts"))
 (gr_line (start 29.16933 19.413215) (end 37.66933 19.413215) (stroke (width 0.2032) (type solid)) (layer "Edge.Cuts"))
 (segment (start 29.91933 23.413215) (end 31.41933 23.413215) (width 0.508) (layer "F.Cu") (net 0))
 (segment (start 36.91933 26.318215) (end 36.91933 25.913215) (width 0.508) (layer "F.Cu") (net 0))
 (segment (start 29.91933 20.508215) (end 29.91933 20.913215) (width 0.508) (layer "F.Cu") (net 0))
 (segment (start 32.47953 26.318215) (end 29.91933 26.318215) (width 0.508) (layer "F.Cu") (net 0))
 (segment (start 36.91933 23.413215) (end 35.41933 23.413215) (width 0.508) (layer "F.Cu") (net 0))
 (segment (start 34.35913 26.318215) (end 36.91933 26.318215) (width 0.508) (layer "F.Cu") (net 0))
 (segment (start 33.41933 22.413215) (end 32.41933 22.413215) (width 0.508) (layer "F.Cu") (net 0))
 (segment (start 36.91933 20.913215) (end 36.91933 21.163215) (width 0.508) (layer "F.Cu") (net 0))
 (segment (start 34.41933 24.413215) (end 33.41933 24.413215) (width 0.508) (layer "F.Cu") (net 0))
 (segment (start 35.41933 23.413215) (end 34.41933 24.413215) (width 0.508) (layer "F.Cu") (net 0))
 (segment (start 36.91933 25.913215) (end 36.91933 26.163215) (width 0.508) (layer "F.Cu") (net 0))
 (segment (start 36.91933 20.508215) (end 36.91933 20.913215) (width 0.508) (layer "F.Cu") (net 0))
 (segment (start 31.41933 23.413215) (end 32.41933 22.413215) (width 0.508) (layer "F.Cu") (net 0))
 (segment (start 29.91933 23.413215) (end 29.66933 23.413215) (width 0.508) (layer "F.Cu") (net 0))
 (segment (start 32.47953 20.508215) (end 29.91933 20.508215) (width 0.508) (layer "F.Cu") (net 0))
 (segment (start 34.35913 20.508215) (end 36.91933 20.508215) (width 0.508) (layer "F.Cu") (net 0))
 (segment (start 29.91933 26.318215) (end 29.91933 25.913215) (width 0.508) (layer "F.Cu") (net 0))
 (segment (start 36.91986 23.42343) (end 37.16986 23.42343) (width 0.508) (layer "B.Cu") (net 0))
 (segment (start 32.26986 21.73593) (end 32.26986 22.47343) (width 0.5) (layer "B.Cu") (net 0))
 (segment (start 29.90736 20.92343) (end 31.45736 20.92343) (width 0.5) (layer "B.Cu") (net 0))
 (segment (start 29.91986 20.51843) (end 29.91986 20.92343) (width 0.508) (layer "B.Cu") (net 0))
 (segment (start 36.91986 20.51843) (end 36.91986 20.92343) (width 0.508) (layer "B.Cu") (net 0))
 (segment (start 32.26986 25.09218) (end 32.26986 24.35468) (width 0.5) (layer "B.Cu") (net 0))
 (segment (start 36.93236 25.92343) (end 35.38236 25.92343) (width 0.5) (layer "B.Cu") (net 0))
 (segment (start 36.91986 26.32843) (end 36.91986 25.92343) (width 0.508) (layer "B.Cu") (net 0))
 (segment (start 31.45736 25.90468) (end 32.26986 25.09218) (width 0.5) (layer "B.Cu") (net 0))
 (segment (start 29.91986 20.92343) (end 29.91986 21.17343) (width 0.508) (layer "B.Cu") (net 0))
 (segment (start 36.91986 20.92343) (end 35.36986 20.92343) (width 0.5) (layer "B.Cu") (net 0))
 (segment (start 34.56986 25.11093) (end 34.56986 24.37343) (width 0.5) (layer "B.Cu") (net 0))
 (segment (start 29.91986 26.32843) (end 29.91986 25.92343) (width 0.508) (layer "B.Cu") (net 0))
 (segment (start 34.55736 23.42343) (end 36.91986 23.42343) (width 0.5) (layer "B.Cu") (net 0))
 (segment (start 34.55736 21.73593) (end 34.55736 22.47343) (width 0.5) (layer "B.Cu") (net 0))
 (segment (start 35.36986 20.92343) (end 34.55736 21.73593) (width 0.5) (layer "B.Cu") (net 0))
 (segment (start 29.90736 25.90468) (end 31.45736 25.90468) (width 0.5) (layer "B.Cu") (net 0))
 (segment (start 32.28236 23.42343) (end 29.91986 23.42343) (width 0.5) (layer "B.Cu") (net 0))
 (segment (start 35.38236 25.92343) (end 34.56986 25.11093) (width 0.5) (layer "B.Cu") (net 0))
 (segment (start 29.91986 25.92343) (end 29.91986 26.17343) (width 0.508) (layer "B.Cu") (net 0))
 (segment (start 31.45736 20.92343) (end 32.26986 21.73593) (width 0.5) (layer "B.Cu") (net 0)))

